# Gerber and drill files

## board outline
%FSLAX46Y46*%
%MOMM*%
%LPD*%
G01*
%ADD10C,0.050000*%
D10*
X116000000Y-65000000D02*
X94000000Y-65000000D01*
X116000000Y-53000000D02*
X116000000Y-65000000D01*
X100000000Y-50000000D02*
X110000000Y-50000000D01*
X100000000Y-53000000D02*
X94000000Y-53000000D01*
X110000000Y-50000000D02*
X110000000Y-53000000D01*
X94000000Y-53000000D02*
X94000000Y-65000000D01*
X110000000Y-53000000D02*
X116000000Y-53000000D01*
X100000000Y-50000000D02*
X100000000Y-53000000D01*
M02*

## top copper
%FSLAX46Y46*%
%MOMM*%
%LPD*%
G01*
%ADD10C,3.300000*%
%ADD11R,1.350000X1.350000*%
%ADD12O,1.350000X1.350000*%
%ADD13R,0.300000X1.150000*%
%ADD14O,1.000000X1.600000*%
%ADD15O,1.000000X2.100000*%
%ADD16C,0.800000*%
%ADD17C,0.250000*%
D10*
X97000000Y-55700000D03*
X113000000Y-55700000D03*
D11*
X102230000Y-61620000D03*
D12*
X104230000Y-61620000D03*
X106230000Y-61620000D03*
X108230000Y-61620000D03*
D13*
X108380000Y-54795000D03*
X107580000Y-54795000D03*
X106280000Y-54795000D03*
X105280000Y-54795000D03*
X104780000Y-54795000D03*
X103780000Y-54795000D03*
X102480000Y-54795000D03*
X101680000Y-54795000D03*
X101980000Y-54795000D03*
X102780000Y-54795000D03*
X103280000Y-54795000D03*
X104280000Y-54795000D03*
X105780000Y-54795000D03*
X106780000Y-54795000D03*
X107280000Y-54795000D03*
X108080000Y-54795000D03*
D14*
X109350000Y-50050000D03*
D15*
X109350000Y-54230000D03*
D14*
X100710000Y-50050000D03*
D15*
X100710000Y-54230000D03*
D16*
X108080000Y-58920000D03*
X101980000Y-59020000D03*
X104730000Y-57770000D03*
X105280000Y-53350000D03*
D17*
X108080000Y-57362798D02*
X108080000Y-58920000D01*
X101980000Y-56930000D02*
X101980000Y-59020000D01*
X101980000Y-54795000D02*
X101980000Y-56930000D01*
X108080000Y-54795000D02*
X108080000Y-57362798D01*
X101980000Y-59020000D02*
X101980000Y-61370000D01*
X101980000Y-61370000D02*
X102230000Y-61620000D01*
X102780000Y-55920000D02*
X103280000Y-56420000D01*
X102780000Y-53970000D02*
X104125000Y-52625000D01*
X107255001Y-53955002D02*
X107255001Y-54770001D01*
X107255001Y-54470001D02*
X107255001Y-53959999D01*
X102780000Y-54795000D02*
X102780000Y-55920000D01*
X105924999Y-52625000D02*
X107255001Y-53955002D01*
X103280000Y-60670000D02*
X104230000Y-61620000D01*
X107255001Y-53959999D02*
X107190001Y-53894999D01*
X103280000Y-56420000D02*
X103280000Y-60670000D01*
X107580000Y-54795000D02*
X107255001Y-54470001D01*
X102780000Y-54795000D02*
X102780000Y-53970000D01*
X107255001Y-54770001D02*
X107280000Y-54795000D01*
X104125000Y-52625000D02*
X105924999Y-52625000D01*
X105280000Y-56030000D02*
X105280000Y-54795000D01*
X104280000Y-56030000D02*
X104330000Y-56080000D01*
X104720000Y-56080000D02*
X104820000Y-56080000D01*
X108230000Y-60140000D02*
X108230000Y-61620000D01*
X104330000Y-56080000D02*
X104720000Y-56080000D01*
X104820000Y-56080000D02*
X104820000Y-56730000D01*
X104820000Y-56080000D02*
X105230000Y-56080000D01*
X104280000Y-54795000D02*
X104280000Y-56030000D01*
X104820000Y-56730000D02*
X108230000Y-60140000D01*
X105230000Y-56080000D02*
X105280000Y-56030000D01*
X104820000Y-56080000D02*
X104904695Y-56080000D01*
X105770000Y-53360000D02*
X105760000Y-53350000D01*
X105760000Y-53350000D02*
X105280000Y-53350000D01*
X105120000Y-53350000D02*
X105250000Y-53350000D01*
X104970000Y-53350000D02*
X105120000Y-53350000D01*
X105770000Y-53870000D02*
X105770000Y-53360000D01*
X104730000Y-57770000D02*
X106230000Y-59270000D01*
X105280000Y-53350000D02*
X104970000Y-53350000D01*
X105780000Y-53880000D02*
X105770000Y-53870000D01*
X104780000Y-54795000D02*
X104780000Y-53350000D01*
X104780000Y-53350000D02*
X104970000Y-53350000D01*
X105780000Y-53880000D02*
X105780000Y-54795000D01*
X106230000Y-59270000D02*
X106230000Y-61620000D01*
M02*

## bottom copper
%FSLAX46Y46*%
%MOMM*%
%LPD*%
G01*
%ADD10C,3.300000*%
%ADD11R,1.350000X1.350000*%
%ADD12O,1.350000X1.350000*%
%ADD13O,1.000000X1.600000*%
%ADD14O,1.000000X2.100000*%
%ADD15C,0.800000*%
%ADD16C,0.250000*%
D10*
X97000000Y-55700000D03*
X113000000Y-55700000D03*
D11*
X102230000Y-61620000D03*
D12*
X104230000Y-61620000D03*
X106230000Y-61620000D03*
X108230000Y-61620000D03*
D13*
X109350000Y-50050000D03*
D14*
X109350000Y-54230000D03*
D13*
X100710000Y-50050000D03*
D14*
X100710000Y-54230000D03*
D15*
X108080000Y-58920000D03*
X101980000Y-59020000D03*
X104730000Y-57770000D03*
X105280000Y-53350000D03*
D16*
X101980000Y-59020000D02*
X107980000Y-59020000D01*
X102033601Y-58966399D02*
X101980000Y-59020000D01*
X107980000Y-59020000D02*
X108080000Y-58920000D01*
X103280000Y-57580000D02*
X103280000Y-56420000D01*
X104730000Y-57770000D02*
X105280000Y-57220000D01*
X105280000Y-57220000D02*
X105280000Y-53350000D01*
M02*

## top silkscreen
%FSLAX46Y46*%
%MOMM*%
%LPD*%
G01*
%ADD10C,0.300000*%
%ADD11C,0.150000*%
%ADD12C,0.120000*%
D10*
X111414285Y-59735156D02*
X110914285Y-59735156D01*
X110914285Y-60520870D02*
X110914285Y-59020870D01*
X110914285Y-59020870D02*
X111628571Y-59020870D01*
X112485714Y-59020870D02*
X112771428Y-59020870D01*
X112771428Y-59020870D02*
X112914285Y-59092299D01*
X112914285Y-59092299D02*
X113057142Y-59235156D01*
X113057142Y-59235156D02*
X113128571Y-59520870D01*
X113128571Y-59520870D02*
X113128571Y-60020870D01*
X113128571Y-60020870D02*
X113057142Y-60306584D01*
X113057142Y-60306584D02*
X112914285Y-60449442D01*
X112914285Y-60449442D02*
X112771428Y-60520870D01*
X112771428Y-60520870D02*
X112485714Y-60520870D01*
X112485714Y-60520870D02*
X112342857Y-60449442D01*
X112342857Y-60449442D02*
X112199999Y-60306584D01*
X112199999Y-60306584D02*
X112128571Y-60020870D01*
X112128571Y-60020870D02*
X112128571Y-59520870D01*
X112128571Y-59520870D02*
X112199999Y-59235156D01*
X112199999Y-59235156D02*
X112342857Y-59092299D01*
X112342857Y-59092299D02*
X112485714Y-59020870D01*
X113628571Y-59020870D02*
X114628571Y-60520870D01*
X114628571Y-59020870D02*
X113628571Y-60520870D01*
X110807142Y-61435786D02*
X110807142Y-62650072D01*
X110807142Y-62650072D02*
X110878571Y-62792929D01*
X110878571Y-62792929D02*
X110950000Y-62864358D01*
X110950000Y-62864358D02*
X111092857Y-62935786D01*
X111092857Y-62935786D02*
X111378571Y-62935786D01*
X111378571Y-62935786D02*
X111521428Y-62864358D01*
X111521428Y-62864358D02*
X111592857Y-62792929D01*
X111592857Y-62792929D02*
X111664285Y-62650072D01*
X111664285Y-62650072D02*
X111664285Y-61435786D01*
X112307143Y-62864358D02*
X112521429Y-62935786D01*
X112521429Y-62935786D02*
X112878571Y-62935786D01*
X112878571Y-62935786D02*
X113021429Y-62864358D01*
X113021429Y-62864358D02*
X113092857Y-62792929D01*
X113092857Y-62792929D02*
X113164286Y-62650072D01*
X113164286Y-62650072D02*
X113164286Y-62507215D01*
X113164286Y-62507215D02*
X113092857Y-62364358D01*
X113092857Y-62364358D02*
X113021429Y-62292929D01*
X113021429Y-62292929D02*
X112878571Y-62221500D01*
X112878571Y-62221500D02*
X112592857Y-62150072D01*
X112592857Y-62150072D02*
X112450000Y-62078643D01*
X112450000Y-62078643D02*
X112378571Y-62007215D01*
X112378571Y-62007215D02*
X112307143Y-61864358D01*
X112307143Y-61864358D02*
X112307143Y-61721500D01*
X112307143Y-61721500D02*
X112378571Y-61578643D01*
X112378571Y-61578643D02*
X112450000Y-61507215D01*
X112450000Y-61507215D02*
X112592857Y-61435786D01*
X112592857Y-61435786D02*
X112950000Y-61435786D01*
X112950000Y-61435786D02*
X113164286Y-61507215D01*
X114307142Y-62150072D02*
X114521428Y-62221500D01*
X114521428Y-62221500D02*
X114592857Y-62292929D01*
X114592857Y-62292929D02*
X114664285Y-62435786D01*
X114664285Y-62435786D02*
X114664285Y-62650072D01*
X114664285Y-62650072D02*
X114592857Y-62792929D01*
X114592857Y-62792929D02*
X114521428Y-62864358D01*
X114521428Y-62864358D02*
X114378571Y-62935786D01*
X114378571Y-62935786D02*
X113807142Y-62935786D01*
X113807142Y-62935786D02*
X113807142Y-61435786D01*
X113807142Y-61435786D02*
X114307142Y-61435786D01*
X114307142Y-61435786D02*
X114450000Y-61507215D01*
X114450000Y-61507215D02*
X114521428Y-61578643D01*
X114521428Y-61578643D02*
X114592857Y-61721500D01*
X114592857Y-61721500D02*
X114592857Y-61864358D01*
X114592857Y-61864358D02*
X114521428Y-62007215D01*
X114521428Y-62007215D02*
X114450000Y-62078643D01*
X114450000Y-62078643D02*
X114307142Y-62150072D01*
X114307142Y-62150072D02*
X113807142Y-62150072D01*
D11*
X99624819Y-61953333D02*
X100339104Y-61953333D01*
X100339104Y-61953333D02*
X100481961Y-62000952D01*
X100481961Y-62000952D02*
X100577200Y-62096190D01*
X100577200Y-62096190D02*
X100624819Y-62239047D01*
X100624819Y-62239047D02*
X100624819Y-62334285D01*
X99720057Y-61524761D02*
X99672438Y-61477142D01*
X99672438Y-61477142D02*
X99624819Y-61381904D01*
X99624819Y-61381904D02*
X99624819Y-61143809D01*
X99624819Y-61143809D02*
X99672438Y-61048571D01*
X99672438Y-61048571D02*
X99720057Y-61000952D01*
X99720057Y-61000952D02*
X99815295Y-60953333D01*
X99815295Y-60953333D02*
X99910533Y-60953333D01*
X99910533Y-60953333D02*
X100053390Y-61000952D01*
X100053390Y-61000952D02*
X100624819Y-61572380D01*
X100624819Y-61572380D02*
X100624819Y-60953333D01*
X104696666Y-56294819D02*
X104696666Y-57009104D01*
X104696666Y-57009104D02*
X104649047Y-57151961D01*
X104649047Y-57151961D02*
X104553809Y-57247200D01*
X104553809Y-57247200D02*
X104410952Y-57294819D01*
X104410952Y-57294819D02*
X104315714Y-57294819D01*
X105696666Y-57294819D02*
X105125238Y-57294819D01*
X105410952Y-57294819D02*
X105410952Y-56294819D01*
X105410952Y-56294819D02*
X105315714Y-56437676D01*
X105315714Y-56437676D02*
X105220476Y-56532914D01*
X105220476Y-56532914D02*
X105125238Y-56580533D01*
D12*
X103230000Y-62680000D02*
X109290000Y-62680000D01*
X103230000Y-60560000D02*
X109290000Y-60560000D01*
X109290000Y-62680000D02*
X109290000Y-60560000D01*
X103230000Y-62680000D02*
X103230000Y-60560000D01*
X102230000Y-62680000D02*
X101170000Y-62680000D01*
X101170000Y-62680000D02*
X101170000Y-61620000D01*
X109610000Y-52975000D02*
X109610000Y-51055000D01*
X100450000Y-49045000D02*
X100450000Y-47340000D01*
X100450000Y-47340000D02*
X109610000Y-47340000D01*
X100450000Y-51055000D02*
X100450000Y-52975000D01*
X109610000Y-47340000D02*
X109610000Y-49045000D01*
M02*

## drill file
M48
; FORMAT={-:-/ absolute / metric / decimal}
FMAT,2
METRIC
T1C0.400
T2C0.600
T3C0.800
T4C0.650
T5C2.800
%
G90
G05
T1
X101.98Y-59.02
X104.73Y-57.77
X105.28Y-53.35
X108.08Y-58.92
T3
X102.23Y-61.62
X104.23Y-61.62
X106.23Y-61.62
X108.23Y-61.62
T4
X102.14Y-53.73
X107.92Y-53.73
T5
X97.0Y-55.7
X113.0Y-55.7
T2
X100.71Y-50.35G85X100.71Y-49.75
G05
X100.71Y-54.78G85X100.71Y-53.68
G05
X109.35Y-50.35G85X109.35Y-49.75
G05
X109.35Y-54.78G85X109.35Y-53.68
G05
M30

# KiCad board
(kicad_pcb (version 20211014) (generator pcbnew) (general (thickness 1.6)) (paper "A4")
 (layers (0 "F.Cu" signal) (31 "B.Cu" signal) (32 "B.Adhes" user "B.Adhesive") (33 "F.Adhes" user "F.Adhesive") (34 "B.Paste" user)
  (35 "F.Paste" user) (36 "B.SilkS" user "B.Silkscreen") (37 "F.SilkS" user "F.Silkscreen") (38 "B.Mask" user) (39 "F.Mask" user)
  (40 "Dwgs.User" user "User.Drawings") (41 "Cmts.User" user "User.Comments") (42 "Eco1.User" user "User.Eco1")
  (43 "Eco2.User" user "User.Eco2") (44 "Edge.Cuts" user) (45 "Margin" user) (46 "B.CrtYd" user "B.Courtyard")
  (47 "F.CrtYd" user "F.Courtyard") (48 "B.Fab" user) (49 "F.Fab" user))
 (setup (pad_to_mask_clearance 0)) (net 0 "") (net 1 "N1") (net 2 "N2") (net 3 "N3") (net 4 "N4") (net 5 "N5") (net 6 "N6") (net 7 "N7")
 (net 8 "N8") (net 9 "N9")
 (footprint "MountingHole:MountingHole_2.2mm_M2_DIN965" (layer "F.Cu") (at 97 55.7)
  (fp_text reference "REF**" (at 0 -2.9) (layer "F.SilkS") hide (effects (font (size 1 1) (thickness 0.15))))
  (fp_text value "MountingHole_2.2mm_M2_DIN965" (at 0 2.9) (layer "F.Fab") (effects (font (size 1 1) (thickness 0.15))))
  (pad "" np_thru_hole circle locked (at 0 0) (size 3.3 3.3) (drill 2.8) (layers F&B.Cu *.Mask)))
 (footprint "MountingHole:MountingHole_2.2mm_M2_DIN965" (layer "F.Cu") (at 113 55.7)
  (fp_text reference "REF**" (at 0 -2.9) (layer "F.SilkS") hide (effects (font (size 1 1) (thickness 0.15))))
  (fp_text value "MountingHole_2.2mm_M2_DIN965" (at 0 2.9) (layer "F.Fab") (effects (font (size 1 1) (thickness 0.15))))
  (pad "" np_thru_hole circle locked (at 0 0 4) (size 3.3 3.3) (drill 2.8) (layers F&B.Cu *.Mask)))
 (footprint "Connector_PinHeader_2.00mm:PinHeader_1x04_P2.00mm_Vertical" (layer "F.Cu") (at 102.23 61.62 90)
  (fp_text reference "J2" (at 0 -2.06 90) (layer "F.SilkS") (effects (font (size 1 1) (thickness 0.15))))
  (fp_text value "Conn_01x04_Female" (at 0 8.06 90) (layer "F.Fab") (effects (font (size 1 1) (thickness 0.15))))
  (fp_line (start -1.06 1) (end -1.06 7.06) (layer "F.SilkS") (width 0.12))
  (fp_line (start 1.06 1) (end 1.06 7.06) (layer "F.SilkS") (width 0.12))
  (fp_line (start -1.06 7.06) (end 1.06 7.06) (layer "F.SilkS") (width 0.12))
  (fp_line (start -1.06 1) (end 1.06 1) (layer "F.SilkS") (width 0.12))
  (fp_line (start -1.06 0) (end -1.06 -1.06) (layer "F.SilkS") (width 0.12))
  (fp_line (start -1.06 -1.06) (end 0 -1.06) (layer "F.SilkS") (width 0.12))
  (pad "1" thru_hole rect (at 0 0 90) (size 1.35 1.35) (drill 0.8) (layers *.Cu *.Mask) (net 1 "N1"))
  (pad "2" thru_hole oval (at 0 2 90) (size 1.35 1.35) (drill 0.8) (layers *.Cu *.Mask) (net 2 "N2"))
  (pad "3" thru_hole oval (at 0 4 90) (size 1.35 1.35) (drill 0.8) (layers *.Cu *.Mask) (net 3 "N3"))
  (pad "4" thru_hole oval (at 0 6 90) (size 1.35 1.35) (drill 0.8) (layers *.Cu *.Mask) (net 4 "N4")))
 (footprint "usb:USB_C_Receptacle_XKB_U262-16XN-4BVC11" (layer "F.Cu") (at 105.03 51.125 180)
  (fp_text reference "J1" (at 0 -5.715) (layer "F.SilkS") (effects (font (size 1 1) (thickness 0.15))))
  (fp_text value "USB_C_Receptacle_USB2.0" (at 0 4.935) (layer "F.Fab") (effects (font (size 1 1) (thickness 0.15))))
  (fp_line (start -4.58 -1.85) (end -4.58 0.07) (layer "F.SilkS") (width 0.12))
  (fp_line (start 4.58 2.08) (end 4.58 3.785) (layer "F.SilkS") (width 0.12))
  (fp_line (start 4.58 3.785) (end -4.58 3.785) (layer "F.SilkS") (width 0.12))
  (fp_line (start 4.58 0.07) (end 4.58 -1.85) (layer "F.SilkS") (width 0.12))
  (fp_line (start -4.58 3.785) (end -4.58 2.08) (layer "F.SilkS") (width 0.12))
  (pad "" np_thru_hole circle locked (at 2.89 -2.605 180) (size 0.65 0.65) (drill 0.65) (layers *.Cu *.Mask))
  (pad "" np_thru_hole circle locked (at -2.89 -2.605 180) (size 0.65 0.65) (drill 0.65) (layers *.Cu *.Mask))
  (pad "A1" smd rect locked (at -3.35 -3.67 180) (size 0.3 1.15) (layers "F.Cu" "F.Paste" "F.Mask") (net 1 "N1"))
  (pad "A4" smd rect locked (at -2.55 -3.67 180) (size 0.3 1.15) (layers "F.Cu" "F.Paste" "F.Mask") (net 2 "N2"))
  (pad "A5" smd rect locked (at -1.25 -3.67 180) (size 0.3 1.15) (layers "F.Cu" "F.Paste" "F.Mask") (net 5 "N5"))
  (pad "A6" smd rect locked (at -0.25 -3.67 180) (size 0.3 1.15) (layers "F.Cu" "F.Paste" "F.Mask") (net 4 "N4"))
  (pad "A7" smd rect locked (at 0.25 -3.67 180) (size 0.3 1.15) (layers "F.Cu" "F.Paste" "F.Mask") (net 3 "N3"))
  (pad "A8" smd rect locked (at 1.25 -3.67 180) (size 0.3 1.15) (layers "F.Cu" "F.Paste" "F.Mask") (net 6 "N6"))
  (pad "A9" smd rect locked (at 2.55 -3.67 180) (size 0.3 1.15) (layers "F.Cu" "F.Paste" "F.Mask") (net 2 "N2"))
  (pad "A12" smd rect locked (at 3.35 -3.67 180) (size 0.3 1.15) (layers "F.Cu" "F.Paste" "F.Mask") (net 1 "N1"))
  (pad "B1" smd rect locked (at 3.05 -3.67 180) (size 0.3 1.15) (layers "F.Cu" "F.Paste" "F.Mask") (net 1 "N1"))
  (pad "B4" smd rect locked (at 2.25 -3.67 180) (size 0.3 1.15) (layers "F.Cu" "F.Paste" "F.Mask") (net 2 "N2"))
  (pad "B5" smd rect locked (at 1.75 -3.67 180) (size 0.3 1.15) (layers "F.Cu" "F.Paste" "F.Mask") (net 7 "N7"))
  (pad "B6" smd rect locked (at 0.75 -3.67 180) (size 0.3 1.15) (layers "F.Cu" "F.Paste" "F.Mask") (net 4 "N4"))
  (pad "B7" smd rect locked (at -0.75 -3.67 180) (size 0.3 1.15) (layers "F.Cu" "F.Paste" "F.Mask") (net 3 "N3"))
  (pad "B8" smd rect locked (at -1.75 -3.67 180) (size 0.3 1.15) (layers "F.Cu" "F.Paste" "F.Mask") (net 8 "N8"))
  (pad "B9" smd rect locked (at -2.25 -3.67 180) (size 0.3 1.15) (layers "F.Cu" "F.Paste" "F.Mask") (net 2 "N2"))
  (pad "B12" smd rect locked (at -3.05 -3.67 180) (size 0.3 1.15) (layers "F.Cu" "F.Paste" "F.Mask") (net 1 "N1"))
  (pad "S1" thru_hole oval locked (at -4.32 1.075 180) (size 1 1.6) (drill oval 0.6 1.2) (layers *.Cu *.Mask) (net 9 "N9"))
  (pad "S1" thru_hole oval locked (at -4.32 -3.105 180) (size 1 2.1) (drill oval 0.6 1.7) (layers *.Cu *.Mask) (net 9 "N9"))
  (pad "S1" thru_hole oval locked (at 4.32 1.075 180) (size 1 1.6) (drill oval 0.6 1.2) (layers *.Cu *.Mask) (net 9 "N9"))
  (pad "S1" thru_hole oval locked (at 4.32 -3.105 180) (size 1 2.1) (drill oval 0.6 1.7) (layers *.Cu *.Mask) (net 9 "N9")))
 (gr_line (start 116 65) (end 94 65) (layer "Edge.Cuts") (width 0.05))
 (gr_line (start 116 53) (end 116 65) (layer "Edge.Cuts") (width 0.05))
 (gr_line (start 100 50) (end 110 50) (layer "Edge.Cuts") (width 0.05))
 (gr_line (start 100 53) (end 94 53) (layer "Edge.Cuts") (width 0.05))
 (gr_line (start 110 50) (end 110 53) (layer "Edge.Cuts") (width 0.05))
 (gr_line (start 94 53) (end 94 65) (layer "Edge.Cuts") (width 0.05))
 (gr_line (start 110 53) (end 116 53) (layer "Edge.Cuts") (width 0.05))
 (gr_line (start 100 50) (end 100 53) (layer "Edge.Cuts") (width 0.05))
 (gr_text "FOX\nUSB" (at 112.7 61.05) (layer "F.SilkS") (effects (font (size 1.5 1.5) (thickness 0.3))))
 (segment (start 108.08 57.362798) (end 108.08 58.92) (width 0.25) (layer "F.Cu") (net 1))
 (segment (start 101.98 56.93) (end 101.98 59.02) (width 0.25) (layer "F.Cu") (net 1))
 (segment (start 101.98 54.795) (end 101.98 56.93) (width 0.25) (layer "F.Cu") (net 1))
 (segment (start 108.08 54.795) (end 108.08 57.362798) (width 0.25) (layer "F.Cu") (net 1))
 (segment (start 101.98 59.02) (end 101.98 61.37) (width 0.25) (layer "F.Cu") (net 1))
 (segment (start 101.98 61.37) (end 102.23 61.62) (width 0.25) (layer "F.Cu") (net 1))
 (via (at 108.08 58.92) (size 0.8) (drill 0.4) (layers "F.Cu" "B.Cu") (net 1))
 (via (at 101.98 59.02) (size 0.8) (drill 0.4) (layers "F.Cu" "B.Cu") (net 1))
 (segment (start 101.98 59.02) (end 107.98 59.02) (width 0.25) (layer "B.Cu") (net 1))
 (segment (start 102.033601 58.966399) (end 101.98 59.02) (width 0.25) (layer "B.Cu") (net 1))
 (segment (start 107.98 59.02) (end 108.08 58.92) (width 0.25) (layer "B.Cu") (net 1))
 (segment (start 102.78 55.92) (end 103.28 56.42) (width 0.25) (layer "F.Cu") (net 2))
 (segment (start 102.78 53.97) (end 104.125 52.625) (width 0.25) (layer "F.Cu") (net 2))
 (segment (start 107.255001 53.955002) (end 107.255001 54.770001) (width 0.25) (layer "F.Cu") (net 2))
 (segment (start 107.255001 54.470001) (end 107.255001 53.959999) (width 0.25) (layer "F.Cu") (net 2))
 (segment (start 102.78 54.795) (end 102.78 55.92) (width 0.25) (layer "F.Cu") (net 2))
 (segment (start 105.924999 52.625) (end 107.255001 53.955002) (width 0.25) (layer "F.Cu") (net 2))
 (segment (start 103.28 60.67) (end 104.23 61.62) (width 0.25) (layer "F.Cu") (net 2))
 (segment (start 107.255001 53.959999) (end 107.190001 53.894999) (width 0.25) (layer "F.Cu") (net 2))
 (segment (start 103.28 56.42) (end 103.28 60.67) (width 0.25) (layer "F.Cu") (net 2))
 (segment (start 107.58 54.795) (end 107.255001 54.470001) (width 0.25) (layer "F.Cu") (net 2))
 (segment (start 102.78 54.795) (end 102.78 53.97) (width 0.25) (layer "F.Cu") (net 2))
 (segment (start 107.255001 54.770001) (end 107.28 54.795) (width 0.25) (layer "F.Cu") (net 2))
 (segment (start 104.125 52.625) (end 105.924999 52.625) (width 0.25) (layer "F.Cu") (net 2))
 (segment (start 103.28 57.58) (end 103.28 56.42) (width 0.25) (layer "B.Cu") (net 5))
 (segment (start 105.28 56.03) (end 105.28 54.795) (width 0.25) (layer "F.Cu") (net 4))
 (segment (start 104.28 56.03) (end 104.33 56.08) (width 0.25) (layer "F.Cu") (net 4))
 (segment (start 104.72 56.08) (end 104.82 56.08) (width 0.25) (layer "F.Cu") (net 4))
 (segment (start 108.23 60.14) (end 108.23 61.62) (width 0.25) (layer "F.Cu") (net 4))
 (segment (start 104.33 56.08) (end 104.72 56.08) (width 0.25) (layer "F.Cu") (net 4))
 (segment (start 104.82 56.08) (end 104.82 56.73) (width 0.25) (layer "F.Cu") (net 4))
 (segment (start 104.82 56.08) (end 105.23 56.08) (width 0.25) (layer "F.Cu") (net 4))
 (segment (start 104.28 54.795) (end 104.28 56.03) (width 0.25) (layer "F.Cu") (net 4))
 (segment (start 104.82 56.73) (end 108.23 60.14) (width 0.25) (layer "F.Cu") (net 4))
 (segment (start 105.23 56.08) (end 105.28 56.03) (width 0.25) (layer "F.Cu") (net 4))
 (segment (start 104.82 56.08) (end 104.904695 56.08) (width 0.25) (layer "F.Cu") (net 4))
 (segment (start 105.77 53.36) (end 105.76 53.35) (width 0.25) (layer "F.Cu") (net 3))
 (segment (start 105.76 53.35) (end 105.28 53.35) (width 0.25) (layer "F.Cu") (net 3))
 (segment (start 105.12 53.35) (end 105.25 53.35) (width 0.25) (layer "F.Cu") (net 3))
 (segment (start 104.97 53.35) (end 105.12 53.35) (width 0.25) (layer "F.Cu") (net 3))
 (segment (start 105.77 53.87) (end 105.77 53.36) (width 0.25) (layer "F.Cu") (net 3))
 (segment (start 104.73 57.77) (end 106.23 59.27) (width 0.25) (layer "F.Cu") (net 3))
 (segment (start 105.28 53.35) (end 104.97 53.35) (width 0.25) (layer "F.Cu") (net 3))
 (segment (start 105.78 53.88) (end 105.77 53.87) (width 0.25) (layer "F.Cu") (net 3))
 (segment (start 104.78 54.795) (end 104.78 53.35) (width 0.25) (layer "F.Cu") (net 3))
 (segment (start 104.78 53.35) (end 104.97 53.35) (width 0.25) (layer "F.Cu") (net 3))
 (segment (start 105.78 53.88) (end 105.78 54.795) (width 0.25) (layer "F.Cu") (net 3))
 (segment (start 106.23 59.27) (end 106.23 61.62) (width 0.25) (layer "F.Cu") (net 3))
 (via (at 104.73 57.77) (size 0.8) (drill 0.4) (layers "F.Cu" "B.Cu") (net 3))
 (via (at 105.28 53.35) (size 0.8) (drill 0.4) (layers "F.Cu" "B.Cu") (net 3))
 (segment (start 104.73 57.77) (end 105.28 57.22) (width 0.25) (layer "B.Cu") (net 3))
 (segment (start 105.28 57.22) (end 105.28 53.35) (width 0.25) (layer "B.Cu") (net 3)))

